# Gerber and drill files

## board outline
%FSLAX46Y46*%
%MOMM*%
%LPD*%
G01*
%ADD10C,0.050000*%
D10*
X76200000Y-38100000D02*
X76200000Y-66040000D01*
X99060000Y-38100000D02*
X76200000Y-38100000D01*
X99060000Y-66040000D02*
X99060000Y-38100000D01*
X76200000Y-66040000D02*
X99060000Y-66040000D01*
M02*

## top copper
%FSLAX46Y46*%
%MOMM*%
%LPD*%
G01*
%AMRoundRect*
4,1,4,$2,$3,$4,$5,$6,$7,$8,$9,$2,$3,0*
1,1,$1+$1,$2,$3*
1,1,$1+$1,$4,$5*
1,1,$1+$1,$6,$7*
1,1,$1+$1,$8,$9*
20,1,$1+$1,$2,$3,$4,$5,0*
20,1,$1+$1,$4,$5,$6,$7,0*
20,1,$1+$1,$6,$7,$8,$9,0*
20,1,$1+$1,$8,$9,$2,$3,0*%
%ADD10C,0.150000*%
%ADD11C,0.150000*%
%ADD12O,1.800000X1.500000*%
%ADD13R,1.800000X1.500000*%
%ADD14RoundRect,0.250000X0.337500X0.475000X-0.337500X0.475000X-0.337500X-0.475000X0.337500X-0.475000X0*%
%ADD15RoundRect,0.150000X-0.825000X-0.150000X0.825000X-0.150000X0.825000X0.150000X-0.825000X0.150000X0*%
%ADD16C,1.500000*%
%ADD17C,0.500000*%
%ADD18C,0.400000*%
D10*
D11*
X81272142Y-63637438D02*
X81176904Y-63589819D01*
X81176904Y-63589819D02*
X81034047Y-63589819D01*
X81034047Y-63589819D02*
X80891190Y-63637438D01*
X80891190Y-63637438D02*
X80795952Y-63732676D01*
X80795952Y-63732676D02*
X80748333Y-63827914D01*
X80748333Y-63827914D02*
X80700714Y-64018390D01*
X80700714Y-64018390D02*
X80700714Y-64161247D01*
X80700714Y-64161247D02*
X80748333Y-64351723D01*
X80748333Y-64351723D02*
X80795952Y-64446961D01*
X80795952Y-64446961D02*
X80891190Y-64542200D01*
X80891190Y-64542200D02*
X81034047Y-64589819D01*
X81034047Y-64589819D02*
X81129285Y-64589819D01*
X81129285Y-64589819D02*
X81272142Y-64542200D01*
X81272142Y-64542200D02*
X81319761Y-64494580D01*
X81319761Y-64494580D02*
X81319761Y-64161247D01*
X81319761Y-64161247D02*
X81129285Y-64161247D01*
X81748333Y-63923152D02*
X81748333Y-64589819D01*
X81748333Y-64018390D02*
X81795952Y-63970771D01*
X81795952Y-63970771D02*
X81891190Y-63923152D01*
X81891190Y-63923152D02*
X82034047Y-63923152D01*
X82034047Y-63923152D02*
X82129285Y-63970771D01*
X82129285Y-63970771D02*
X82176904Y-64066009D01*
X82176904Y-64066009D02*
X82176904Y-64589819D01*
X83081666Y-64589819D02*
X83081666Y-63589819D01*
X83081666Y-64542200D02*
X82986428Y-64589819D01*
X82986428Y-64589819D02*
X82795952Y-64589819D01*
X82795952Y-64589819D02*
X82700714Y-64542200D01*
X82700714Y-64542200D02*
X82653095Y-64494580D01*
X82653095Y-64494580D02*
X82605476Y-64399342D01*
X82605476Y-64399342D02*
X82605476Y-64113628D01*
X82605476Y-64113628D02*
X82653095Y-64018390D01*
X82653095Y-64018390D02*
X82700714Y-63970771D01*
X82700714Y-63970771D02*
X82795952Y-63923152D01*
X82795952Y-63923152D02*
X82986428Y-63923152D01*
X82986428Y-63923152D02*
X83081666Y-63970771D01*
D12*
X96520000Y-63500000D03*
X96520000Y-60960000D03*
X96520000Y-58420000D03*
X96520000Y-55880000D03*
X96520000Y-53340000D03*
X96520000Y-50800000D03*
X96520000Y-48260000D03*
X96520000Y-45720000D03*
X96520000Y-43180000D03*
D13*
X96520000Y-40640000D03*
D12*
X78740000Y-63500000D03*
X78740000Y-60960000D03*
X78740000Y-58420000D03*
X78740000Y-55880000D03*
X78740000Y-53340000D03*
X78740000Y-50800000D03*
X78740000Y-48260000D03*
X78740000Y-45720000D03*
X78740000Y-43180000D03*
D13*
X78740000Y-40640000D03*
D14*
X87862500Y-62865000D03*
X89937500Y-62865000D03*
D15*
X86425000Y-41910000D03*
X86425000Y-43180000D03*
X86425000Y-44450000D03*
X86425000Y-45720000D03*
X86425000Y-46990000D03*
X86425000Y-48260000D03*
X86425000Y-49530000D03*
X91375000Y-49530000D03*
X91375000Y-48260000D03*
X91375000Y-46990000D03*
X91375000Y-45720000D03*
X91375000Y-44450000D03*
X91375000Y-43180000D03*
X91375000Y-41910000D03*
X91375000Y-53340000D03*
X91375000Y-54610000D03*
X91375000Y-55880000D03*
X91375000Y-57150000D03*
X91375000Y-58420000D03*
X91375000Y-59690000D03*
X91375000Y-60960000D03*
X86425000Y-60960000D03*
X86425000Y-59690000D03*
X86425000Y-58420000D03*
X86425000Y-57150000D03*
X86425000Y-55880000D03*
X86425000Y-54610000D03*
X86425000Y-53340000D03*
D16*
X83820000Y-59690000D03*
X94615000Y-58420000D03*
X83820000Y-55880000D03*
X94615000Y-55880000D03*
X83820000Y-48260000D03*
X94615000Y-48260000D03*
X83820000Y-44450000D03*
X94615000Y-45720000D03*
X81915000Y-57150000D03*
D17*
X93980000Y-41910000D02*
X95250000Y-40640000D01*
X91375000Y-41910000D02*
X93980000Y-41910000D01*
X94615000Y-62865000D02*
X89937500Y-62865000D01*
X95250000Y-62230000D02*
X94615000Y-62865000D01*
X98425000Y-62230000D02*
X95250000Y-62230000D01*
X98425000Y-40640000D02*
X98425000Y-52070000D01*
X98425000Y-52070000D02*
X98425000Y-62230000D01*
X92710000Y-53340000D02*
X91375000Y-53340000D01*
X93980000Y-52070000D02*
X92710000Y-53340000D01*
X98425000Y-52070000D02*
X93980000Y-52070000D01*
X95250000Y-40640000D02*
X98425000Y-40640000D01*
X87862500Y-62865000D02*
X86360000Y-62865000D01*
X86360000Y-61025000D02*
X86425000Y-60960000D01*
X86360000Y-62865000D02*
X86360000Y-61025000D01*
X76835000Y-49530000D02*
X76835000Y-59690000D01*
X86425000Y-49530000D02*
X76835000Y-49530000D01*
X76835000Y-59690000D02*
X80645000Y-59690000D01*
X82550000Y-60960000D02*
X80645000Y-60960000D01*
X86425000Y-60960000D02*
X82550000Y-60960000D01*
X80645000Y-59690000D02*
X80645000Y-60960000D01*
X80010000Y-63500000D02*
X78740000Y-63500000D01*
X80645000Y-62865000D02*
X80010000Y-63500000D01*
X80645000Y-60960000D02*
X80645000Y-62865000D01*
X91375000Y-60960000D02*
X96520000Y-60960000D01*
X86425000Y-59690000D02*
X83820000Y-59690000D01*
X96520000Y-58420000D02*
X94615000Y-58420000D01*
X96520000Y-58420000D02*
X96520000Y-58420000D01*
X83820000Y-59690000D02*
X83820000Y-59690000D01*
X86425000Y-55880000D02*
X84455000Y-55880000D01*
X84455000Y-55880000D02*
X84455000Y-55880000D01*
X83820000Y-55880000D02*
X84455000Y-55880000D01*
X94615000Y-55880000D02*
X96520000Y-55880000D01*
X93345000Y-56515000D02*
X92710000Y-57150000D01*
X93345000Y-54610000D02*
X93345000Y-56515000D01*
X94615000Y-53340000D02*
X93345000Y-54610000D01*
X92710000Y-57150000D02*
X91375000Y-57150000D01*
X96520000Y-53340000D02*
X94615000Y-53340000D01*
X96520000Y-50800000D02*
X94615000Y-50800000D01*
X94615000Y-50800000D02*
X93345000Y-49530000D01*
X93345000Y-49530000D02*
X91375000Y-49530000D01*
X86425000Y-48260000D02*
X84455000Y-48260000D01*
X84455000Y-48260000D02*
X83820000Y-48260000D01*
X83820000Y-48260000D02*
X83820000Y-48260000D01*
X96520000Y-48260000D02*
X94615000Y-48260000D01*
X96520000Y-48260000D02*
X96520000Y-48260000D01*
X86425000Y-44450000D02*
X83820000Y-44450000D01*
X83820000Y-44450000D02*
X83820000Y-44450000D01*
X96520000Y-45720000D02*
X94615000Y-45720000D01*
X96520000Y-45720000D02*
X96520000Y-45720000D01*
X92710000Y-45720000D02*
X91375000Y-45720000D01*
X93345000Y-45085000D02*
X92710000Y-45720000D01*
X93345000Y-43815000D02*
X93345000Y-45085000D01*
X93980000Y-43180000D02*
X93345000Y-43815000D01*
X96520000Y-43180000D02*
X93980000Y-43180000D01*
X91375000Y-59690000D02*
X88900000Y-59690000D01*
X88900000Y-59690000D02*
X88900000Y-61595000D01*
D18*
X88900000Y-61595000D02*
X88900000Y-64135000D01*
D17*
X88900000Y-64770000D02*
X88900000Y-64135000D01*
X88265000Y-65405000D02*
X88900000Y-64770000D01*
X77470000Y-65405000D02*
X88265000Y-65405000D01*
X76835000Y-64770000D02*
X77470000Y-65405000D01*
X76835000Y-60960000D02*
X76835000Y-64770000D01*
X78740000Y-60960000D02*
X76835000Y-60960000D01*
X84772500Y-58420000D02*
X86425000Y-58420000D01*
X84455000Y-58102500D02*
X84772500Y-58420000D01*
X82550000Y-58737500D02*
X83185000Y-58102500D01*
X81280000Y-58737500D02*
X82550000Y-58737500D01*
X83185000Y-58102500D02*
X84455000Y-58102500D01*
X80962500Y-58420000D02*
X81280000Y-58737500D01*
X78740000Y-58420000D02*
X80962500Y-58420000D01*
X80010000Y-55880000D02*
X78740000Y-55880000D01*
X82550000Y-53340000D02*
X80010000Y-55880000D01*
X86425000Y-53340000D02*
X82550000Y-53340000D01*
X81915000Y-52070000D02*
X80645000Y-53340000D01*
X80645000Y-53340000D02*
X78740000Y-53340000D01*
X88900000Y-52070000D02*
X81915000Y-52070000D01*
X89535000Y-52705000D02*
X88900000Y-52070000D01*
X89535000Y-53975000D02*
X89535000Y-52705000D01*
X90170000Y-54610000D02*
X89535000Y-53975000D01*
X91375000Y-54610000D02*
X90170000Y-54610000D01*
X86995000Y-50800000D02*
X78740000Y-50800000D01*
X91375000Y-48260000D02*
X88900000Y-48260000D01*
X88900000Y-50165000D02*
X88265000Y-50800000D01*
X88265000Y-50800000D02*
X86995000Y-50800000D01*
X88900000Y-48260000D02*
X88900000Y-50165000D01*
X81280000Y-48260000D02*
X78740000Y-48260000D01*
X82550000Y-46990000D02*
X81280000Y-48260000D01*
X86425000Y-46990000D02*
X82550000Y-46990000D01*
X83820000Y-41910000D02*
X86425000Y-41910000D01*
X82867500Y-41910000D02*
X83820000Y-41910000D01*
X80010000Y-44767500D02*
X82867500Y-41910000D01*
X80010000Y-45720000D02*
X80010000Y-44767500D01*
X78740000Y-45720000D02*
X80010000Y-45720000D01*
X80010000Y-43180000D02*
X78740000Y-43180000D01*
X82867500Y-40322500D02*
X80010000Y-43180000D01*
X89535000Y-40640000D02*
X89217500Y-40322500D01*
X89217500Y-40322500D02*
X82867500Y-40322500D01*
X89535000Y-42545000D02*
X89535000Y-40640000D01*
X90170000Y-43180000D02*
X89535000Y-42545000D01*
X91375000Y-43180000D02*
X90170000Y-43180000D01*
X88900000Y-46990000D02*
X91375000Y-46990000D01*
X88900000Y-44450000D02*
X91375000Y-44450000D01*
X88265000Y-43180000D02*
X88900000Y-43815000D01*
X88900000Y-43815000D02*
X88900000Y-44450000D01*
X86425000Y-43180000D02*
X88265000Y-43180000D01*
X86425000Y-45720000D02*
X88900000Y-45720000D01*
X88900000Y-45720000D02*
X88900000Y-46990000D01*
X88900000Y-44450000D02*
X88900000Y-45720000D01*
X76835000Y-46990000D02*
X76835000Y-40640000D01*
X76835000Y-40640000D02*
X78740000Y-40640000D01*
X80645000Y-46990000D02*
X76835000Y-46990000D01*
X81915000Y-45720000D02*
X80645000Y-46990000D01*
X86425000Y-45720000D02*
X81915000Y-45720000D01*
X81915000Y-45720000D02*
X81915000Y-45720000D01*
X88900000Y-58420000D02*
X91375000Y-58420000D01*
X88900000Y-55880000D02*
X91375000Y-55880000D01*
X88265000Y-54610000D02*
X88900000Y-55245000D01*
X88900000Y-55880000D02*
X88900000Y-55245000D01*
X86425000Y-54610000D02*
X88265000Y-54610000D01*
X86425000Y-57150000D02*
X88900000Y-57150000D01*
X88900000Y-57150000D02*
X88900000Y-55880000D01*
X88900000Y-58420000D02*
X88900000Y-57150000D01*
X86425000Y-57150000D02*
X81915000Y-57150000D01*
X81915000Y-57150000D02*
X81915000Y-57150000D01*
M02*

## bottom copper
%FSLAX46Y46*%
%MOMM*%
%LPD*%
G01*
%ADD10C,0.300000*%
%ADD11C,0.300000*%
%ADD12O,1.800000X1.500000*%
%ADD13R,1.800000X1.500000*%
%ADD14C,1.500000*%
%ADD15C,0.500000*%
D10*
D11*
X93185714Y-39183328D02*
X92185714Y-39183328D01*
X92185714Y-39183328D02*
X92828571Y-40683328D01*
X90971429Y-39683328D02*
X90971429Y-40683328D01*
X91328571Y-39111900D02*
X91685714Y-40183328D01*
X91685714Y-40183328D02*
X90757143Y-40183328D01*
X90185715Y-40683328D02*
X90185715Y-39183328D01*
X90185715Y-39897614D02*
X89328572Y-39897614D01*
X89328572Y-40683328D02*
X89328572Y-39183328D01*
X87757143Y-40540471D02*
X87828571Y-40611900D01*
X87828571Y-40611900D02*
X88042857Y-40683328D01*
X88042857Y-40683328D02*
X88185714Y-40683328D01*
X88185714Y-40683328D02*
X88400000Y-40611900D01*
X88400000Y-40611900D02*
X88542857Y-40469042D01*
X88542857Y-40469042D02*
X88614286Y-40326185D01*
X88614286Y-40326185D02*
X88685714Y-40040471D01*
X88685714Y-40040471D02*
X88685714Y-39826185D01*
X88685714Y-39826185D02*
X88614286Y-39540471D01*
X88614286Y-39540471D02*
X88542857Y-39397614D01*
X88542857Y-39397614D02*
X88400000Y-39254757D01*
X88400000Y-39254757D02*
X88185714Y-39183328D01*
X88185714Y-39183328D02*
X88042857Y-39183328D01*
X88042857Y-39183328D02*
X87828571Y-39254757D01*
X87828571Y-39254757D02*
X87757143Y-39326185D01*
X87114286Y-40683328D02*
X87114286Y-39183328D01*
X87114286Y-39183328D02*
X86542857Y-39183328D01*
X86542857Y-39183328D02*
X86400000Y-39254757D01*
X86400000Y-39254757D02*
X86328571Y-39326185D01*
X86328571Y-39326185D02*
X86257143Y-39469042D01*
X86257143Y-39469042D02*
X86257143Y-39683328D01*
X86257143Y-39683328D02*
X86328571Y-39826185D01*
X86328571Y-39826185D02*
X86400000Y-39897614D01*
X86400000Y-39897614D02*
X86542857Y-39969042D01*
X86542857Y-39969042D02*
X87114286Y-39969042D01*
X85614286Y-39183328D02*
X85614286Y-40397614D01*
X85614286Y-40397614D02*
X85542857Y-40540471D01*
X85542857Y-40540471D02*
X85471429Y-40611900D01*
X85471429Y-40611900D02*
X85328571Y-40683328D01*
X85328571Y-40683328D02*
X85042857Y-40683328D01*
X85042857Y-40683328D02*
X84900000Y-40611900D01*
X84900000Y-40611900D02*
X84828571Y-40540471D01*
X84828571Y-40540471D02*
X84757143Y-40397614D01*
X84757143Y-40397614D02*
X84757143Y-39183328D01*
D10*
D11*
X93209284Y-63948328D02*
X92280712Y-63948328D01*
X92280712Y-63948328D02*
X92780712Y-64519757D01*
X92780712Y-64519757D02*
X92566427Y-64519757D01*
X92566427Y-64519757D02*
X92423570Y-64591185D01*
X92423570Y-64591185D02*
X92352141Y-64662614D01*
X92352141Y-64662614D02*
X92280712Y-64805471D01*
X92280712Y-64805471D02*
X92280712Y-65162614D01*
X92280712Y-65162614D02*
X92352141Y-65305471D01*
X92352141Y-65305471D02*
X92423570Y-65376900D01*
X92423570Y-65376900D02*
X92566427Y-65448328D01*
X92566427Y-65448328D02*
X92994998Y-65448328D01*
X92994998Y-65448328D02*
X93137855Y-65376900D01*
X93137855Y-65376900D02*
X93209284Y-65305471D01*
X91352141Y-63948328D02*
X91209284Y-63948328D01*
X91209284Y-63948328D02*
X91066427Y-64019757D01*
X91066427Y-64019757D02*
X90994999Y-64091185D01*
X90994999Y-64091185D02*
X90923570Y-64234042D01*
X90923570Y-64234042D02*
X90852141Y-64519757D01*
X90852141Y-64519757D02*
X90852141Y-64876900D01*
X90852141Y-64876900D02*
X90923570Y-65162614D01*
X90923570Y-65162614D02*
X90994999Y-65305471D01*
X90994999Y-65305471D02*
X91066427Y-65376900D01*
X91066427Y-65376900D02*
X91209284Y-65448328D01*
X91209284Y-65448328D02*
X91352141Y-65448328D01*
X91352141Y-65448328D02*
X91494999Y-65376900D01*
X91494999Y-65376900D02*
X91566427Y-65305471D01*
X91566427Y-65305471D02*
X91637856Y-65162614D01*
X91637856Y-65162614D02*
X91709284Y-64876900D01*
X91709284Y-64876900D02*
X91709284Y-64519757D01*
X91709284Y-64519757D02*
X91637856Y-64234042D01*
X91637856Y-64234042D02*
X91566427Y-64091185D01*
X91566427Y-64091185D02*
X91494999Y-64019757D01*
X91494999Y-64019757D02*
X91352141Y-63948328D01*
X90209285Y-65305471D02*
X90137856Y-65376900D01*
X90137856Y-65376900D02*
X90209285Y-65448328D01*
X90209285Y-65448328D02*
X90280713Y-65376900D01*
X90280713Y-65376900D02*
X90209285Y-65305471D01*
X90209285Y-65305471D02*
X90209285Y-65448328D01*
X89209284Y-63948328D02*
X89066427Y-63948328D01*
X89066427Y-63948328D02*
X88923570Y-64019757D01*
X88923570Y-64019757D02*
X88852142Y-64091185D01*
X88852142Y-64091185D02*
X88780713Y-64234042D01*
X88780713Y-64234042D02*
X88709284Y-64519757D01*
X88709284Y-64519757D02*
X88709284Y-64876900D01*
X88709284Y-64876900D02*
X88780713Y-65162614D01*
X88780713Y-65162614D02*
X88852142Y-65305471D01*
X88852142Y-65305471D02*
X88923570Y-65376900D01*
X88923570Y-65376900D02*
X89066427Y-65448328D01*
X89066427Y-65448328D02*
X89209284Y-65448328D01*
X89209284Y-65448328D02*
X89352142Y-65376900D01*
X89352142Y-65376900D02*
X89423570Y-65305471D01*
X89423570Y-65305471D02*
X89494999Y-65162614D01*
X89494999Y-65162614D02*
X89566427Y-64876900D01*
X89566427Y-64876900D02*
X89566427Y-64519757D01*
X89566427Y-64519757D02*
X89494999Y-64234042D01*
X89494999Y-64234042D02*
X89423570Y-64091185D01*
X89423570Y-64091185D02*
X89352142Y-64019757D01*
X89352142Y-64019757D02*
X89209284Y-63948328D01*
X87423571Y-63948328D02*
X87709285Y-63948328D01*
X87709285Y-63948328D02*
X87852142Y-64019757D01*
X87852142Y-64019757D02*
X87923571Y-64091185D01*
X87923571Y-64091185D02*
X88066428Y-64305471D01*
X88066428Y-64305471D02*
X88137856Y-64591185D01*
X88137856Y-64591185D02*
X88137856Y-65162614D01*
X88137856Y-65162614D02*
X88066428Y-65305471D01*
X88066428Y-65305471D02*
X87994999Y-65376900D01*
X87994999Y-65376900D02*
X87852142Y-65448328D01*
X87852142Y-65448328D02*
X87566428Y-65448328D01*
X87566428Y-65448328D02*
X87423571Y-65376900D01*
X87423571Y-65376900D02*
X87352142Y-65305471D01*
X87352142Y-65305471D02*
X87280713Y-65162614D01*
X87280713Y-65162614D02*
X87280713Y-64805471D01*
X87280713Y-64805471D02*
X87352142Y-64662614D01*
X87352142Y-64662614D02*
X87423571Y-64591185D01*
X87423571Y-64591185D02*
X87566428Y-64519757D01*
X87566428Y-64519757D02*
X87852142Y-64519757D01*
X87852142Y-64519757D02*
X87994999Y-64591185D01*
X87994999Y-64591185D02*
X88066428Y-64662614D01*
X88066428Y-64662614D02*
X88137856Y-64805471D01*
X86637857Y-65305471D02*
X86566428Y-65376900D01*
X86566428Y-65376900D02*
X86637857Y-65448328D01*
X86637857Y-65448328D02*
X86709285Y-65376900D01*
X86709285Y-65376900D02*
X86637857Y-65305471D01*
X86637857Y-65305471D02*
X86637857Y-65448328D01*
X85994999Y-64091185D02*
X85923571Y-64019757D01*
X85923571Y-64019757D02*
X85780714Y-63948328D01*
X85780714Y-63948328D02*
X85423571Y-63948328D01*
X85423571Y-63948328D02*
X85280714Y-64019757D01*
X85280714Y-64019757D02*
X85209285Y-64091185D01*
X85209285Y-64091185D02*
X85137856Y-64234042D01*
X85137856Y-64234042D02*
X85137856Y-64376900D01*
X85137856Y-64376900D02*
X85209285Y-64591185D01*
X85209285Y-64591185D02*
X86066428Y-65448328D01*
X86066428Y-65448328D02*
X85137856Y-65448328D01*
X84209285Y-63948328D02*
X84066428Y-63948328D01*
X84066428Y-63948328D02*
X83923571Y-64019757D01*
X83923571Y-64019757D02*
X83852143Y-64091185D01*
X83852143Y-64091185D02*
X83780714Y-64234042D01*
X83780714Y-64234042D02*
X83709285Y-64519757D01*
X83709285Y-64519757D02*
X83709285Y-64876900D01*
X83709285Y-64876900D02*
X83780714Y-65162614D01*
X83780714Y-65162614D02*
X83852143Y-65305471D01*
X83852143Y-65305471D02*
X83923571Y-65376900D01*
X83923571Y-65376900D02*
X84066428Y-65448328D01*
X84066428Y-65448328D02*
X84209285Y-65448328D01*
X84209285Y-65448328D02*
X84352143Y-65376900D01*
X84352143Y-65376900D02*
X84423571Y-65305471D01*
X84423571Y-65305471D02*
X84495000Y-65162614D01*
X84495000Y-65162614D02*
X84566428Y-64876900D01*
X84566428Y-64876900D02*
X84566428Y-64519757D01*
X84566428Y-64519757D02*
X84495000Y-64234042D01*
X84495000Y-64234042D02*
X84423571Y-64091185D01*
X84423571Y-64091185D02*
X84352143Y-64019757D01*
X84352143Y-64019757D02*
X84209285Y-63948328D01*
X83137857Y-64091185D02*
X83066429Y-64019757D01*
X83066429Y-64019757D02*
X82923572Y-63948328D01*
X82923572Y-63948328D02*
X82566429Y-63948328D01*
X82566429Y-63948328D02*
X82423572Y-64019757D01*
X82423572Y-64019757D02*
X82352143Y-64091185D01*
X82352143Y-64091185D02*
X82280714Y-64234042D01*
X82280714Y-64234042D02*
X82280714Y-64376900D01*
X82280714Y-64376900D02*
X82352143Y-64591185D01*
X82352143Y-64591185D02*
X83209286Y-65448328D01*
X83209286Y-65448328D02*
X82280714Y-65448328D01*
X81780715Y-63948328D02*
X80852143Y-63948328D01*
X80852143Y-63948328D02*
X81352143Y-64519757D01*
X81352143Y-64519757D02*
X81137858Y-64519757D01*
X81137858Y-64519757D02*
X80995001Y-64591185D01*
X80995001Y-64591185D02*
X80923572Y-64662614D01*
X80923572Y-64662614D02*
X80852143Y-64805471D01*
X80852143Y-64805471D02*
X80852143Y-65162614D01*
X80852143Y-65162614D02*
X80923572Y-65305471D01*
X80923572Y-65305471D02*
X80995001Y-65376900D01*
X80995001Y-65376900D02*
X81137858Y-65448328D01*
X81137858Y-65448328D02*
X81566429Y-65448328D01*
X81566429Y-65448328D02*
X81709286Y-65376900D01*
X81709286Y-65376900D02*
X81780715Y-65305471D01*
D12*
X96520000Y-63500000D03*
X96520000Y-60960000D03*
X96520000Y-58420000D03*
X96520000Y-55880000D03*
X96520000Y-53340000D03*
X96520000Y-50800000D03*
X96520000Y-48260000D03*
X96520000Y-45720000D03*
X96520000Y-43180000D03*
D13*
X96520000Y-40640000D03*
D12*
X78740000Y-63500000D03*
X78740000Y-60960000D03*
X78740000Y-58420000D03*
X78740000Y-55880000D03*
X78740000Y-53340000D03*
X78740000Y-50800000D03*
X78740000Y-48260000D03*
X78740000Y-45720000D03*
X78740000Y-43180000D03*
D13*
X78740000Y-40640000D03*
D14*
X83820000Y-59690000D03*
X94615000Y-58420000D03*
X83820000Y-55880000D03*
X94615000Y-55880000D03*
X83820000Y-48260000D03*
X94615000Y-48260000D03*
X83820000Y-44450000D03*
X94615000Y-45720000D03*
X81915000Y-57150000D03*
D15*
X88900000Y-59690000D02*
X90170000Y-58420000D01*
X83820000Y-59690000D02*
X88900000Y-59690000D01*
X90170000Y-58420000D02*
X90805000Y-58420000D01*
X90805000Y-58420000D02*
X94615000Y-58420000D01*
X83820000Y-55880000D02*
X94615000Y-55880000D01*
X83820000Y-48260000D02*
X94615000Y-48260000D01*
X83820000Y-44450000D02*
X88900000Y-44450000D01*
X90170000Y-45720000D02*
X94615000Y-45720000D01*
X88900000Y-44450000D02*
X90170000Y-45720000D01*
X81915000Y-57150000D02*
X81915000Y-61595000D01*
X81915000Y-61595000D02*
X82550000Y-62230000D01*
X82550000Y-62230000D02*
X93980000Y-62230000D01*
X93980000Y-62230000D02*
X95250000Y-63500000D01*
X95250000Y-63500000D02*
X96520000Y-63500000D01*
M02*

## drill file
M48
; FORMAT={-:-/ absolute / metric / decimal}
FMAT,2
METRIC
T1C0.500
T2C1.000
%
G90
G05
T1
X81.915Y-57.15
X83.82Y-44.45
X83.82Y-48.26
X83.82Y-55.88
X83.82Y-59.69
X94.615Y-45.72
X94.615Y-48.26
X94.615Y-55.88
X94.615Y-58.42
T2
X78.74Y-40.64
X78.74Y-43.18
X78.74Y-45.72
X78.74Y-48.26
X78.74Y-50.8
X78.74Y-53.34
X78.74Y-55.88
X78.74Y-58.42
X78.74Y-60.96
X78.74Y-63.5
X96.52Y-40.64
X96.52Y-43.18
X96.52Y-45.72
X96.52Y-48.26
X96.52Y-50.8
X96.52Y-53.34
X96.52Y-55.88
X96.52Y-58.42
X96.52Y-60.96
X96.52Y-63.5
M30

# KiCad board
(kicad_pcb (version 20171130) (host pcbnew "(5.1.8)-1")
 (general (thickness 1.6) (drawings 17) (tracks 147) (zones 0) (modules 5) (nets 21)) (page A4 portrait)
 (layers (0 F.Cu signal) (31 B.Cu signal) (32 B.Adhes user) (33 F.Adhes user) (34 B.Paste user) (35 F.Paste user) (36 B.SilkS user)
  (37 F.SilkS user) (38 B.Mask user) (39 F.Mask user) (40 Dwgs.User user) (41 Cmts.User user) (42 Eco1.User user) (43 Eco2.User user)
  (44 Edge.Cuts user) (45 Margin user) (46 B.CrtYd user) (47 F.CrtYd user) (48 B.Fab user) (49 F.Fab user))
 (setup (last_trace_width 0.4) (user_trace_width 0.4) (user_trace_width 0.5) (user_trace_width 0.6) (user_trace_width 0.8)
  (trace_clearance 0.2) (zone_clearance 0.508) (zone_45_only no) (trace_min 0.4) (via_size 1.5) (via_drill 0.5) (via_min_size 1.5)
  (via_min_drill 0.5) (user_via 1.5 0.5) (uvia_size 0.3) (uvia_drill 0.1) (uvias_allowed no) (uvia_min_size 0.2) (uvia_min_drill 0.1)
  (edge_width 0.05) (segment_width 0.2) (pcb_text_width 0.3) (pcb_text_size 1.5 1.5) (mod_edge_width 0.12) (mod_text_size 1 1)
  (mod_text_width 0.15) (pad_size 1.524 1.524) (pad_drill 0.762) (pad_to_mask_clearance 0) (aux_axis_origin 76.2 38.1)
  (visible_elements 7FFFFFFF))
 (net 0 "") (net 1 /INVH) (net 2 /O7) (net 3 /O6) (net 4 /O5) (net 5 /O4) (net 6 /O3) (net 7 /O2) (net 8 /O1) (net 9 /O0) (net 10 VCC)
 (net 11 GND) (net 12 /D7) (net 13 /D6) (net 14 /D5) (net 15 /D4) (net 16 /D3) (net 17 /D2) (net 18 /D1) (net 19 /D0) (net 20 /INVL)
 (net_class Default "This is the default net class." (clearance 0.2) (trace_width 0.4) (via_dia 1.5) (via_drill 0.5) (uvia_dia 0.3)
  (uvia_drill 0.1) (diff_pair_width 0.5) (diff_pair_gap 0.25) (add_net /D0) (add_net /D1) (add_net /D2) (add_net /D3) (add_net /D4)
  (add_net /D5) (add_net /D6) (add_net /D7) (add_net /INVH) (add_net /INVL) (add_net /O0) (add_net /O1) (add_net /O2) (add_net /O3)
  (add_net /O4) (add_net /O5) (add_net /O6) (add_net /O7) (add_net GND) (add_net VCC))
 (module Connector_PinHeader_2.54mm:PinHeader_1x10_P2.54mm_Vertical (layer B.Cu) (at 96.52 40.64 180)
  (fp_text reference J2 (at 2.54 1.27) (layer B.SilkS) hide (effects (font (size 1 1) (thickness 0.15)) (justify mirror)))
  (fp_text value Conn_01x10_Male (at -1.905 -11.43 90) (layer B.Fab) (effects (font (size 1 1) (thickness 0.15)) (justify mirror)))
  (pad 10 thru_hole oval (at 0 -22.86 180) (size 1.8 1.5) (drill 1) (layers *.Cu *.Mask) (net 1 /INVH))
  (pad 9 thru_hole oval (at 0 -20.32 180) (size 1.8 1.5) (drill 1) (layers *.Cu *.Mask) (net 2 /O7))
  (pad 8 thru_hole oval (at 0 -17.78 180) (size 1.8 1.5) (drill 1) (layers *.Cu *.Mask) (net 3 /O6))
  (pad 7 thru_hole oval (at 0 -15.24 180) (size 1.8 1.5) (drill 1) (layers *.Cu *.Mask) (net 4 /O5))
  (pad 6 thru_hole oval (at 0 -12.7 180) (size 1.8 1.5) (drill 1) (layers *.Cu *.Mask) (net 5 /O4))
  (pad 5 thru_hole oval (at 0 -10.16 180) (size 1.8 1.5) (drill 1) (layers *.Cu *.Mask) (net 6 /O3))
  (pad 4 thru_hole oval (at 0 -7.62 180) (size 1.8 1.5) (drill 1) (layers *.Cu *.Mask) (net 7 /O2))
  (pad 3 thru_hole oval (at 0 -5.08 180) (size 1.8 1.5) (drill 1) (layers *.Cu *.Mask) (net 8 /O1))
  (pad 2 thru_hole oval (at 0 -2.54 180) (size 1.8 1.5) (drill 1) (layers *.Cu *.Mask) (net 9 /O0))
  (pad 1 thru_hole rect (at 0 0 180) (size 1.8 1.5) (drill 1) (layers *.Cu *.Mask) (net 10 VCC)))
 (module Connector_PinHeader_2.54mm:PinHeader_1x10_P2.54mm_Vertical (layer B.Cu) (at 78.74 40.64 180)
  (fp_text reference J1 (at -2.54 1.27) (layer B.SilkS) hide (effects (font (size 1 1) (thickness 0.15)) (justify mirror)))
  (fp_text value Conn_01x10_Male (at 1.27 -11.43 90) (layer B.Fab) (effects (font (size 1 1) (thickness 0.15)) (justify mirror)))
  (pad 10 thru_hole oval (at 0 -22.86 180) (size 1.8 1.5) (drill 1) (layers *.Cu *.Mask) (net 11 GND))
  (pad 9 thru_hole oval (at 0 -20.32 180) (size 1.8 1.5) (drill 1) (layers *.Cu *.Mask) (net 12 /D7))
  (pad 8 thru_hole oval (at 0 -17.78 180) (size 1.8 1.5) (drill 1) (layers *.Cu *.Mask) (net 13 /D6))
  (pad 7 thru_hole oval (at 0 -15.24 180) (size 1.8 1.5) (drill 1) (layers *.Cu *.Mask) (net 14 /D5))
  (pad 6 thru_hole oval (at 0 -12.7 180) (size 1.8 1.5) (drill 1) (layers *.Cu *.Mask) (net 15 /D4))
  (pad 5 thru_hole oval (at 0 -10.16 180) (size 1.8 1.5) (drill 1) (layers *.Cu *.Mask) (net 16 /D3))
  (pad 4 thru_hole oval (at 0 -7.62 180) (size 1.8 1.5) (drill 1) (layers *.Cu *.Mask) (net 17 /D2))
  (pad 3 thru_hole oval (at 0 -5.08 180) (size 1.8 1.5) (drill 1) (layers *.Cu *.Mask) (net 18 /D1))
  (pad 2 thru_hole oval (at 0 -2.54 180) (size 1.8 1.5) (drill 1) (layers *.Cu *.Mask) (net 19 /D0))
  (pad 1 thru_hole rect (at 0 0 180) (size 1.8 1.5) (drill 1) (layers *.Cu *.Mask) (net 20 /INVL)))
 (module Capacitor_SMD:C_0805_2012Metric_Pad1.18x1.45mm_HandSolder (layer F.Cu) (at 88.9 62.865 180)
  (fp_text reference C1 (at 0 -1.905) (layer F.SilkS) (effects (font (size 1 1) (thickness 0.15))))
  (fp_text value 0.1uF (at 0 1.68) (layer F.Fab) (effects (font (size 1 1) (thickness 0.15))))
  (pad 2 smd roundrect (at 1.0375 0 180) (size 1.175 1.45) (layers F.Cu F.Paste F.Mask) (roundrect_rratio 0.2127659574468085) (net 11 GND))
  (pad 1 smd roundrect (at -1.0375 0 180) (size 1.175 1.45) (layers F.Cu F.Paste F.Mask) (roundrect_rratio 0.2127659574468085) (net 10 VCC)))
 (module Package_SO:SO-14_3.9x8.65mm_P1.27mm (layer F.Cu) (at 88.9 45.72)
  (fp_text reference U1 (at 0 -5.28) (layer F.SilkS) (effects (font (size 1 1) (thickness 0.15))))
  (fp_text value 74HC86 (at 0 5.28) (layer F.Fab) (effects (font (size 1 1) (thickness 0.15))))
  (pad 1 smd roundrect (at -2.475 -3.81) (size 1.95 0.6) (layers F.Cu F.Paste F.Mask) (roundrect_rratio 0.25) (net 18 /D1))
  (pad 2 smd roundrect (at -2.475 -2.54) (size 1.95 0.6) (layers F.Cu F.Paste F.Mask) (roundrect_rratio 0.25) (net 20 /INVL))
  (pad 3 smd roundrect (at -2.475 -1.27) (size 1.95 0.6) (layers F.Cu F.Paste F.Mask) (roundrect_rratio 0.25) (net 8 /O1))
  (pad 4 smd roundrect (at -2.475 0) (size 1.95 0.6) (layers F.Cu F.Paste F.Mask) (roundrect_rratio 0.25) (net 20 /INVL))
  (pad 5 smd roundrect (at -2.475 1.27) (size 1.95 0.6) (layers F.Cu F.Paste F.Mask) (roundrect_rratio 0.25) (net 17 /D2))
  (pad 6 smd roundrect (at -2.475 2.54) (size 1.95 0.6) (layers F.Cu F.Paste F.Mask) (roundrect_rratio 0.25) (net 7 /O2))
  (pad 7 smd roundrect (at -2.475 3.81) (size 1.95 0.6) (layers F.Cu F.Paste F.Mask) (roundrect_rratio 0.25) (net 11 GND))
  (pad 8 smd roundrect (at 2.475 3.81) (size 1.95 0.6) (layers F.Cu F.Paste F.Mask) (roundrect_rratio 0.25) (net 6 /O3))
  (pad 9 smd roundrect (at 2.475 2.54) (size 1.95 0.6) (layers F.Cu F.Paste F.Mask) (roundrect_rratio 0.25) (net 16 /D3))
  (pad 10 smd roundrect (at 2.475 1.27) (size 1.95 0.6) (layers F.Cu F.Paste F.Mask) (roundrect_rratio 0.25) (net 20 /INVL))
  (pad 11 smd roundrect (at 2.475 0) (size 1.95 0.6) (layers F.Cu F.Paste F.Mask) (roundrect_rratio 0.25) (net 9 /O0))
  (pad 12 smd roundrect (at 2.475 -1.27) (size 1.95 0.6) (layers F.Cu F.Paste F.Mask) (roundrect_rratio 0.25) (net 20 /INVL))
  (pad 13 smd roundrect (at 2.475 -2.54) (size 1.95 0.6) (layers F.Cu F.Paste F.Mask) (roundrect_rratio 0.25) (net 19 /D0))
  (pad 14 smd roundrect (at 2.475 -3.81) (size 1.95 0.6) (layers F.Cu F.Paste F.Mask) (roundrect_rratio 0.25) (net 10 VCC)))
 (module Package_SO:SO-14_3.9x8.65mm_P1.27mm (layer F.Cu) (at 88.9 57.15)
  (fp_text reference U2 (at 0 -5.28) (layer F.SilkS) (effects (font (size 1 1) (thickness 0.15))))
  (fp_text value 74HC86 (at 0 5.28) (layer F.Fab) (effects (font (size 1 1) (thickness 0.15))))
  (pad 14 smd roundrect (at 2.475 -3.81) (size 1.95 0.6) (layers F.Cu F.Paste F.Mask) (roundrect_rratio 0.25) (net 10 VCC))
  (pad 13 smd roundrect (at 2.475 -2.54) (size 1.95 0.6) (layers F.Cu F.Paste F.Mask) (roundrect_rratio 0.25) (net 15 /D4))
  (pad 12 smd roundrect (at 2.475 -1.27) (size 1.95 0.6) (layers F.Cu F.Paste F.Mask) (roundrect_rratio 0.25) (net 1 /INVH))
  (pad 11 smd roundrect (at 2.475 0) (size 1.95 0.6) (layers F.Cu F.Paste F.Mask) (roundrect_rratio 0.25) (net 5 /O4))
  (pad 10 smd roundrect (at 2.475 1.27) (size 1.95 0.6) (layers F.Cu F.Paste F.Mask) (roundrect_rratio 0.25) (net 1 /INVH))
  (pad 9 smd roundrect (at 2.475 2.54) (size 1.95 0.6) (layers F.Cu F.Paste F.Mask) (roundrect_rratio 0.25) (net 12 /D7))
  (pad 8 smd roundrect (at 2.475 3.81) (size 1.95 0.6) (layers F.Cu F.Paste F.Mask) (roundrect_rratio 0.25) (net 2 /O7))
  (pad 7 smd roundrect (at -2.475 3.81) (size 1.95 0.6) (layers F.Cu F.Paste F.Mask) (roundrect_rratio 0.25) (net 11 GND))
  (pad 6 smd roundrect (at -2.475 2.54) (size 1.95 0.6) (layers F.Cu F.Paste F.Mask) (roundrect_rratio 0.25) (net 3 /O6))
  (pad 5 smd roundrect (at -2.475 1.27) (size 1.95 0.6) (layers F.Cu F.Paste F.Mask) (roundrect_rratio 0.25) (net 13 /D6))
  (pad 4 smd roundrect (at -2.475 0) (size 1.95 0.6) (layers F.Cu F.Paste F.Mask) (roundrect_rratio 0.25) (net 1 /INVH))
  (pad 3 smd roundrect (at -2.475 -1.27) (size 1.95 0.6) (layers F.Cu F.Paste F.Mask) (roundrect_rratio 0.25) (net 4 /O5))
  (pad 2 smd roundrect (at -2.475 -2.54) (size 1.95 0.6) (layers F.Cu F.Paste F.Mask) (roundrect_rratio 0.25) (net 1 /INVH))
  (pad 1 smd roundrect (at -2.475 -3.81) (size 1.95 0.6) (layers F.Cu F.Paste F.Mask) (roundrect_rratio 0.25) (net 14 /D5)))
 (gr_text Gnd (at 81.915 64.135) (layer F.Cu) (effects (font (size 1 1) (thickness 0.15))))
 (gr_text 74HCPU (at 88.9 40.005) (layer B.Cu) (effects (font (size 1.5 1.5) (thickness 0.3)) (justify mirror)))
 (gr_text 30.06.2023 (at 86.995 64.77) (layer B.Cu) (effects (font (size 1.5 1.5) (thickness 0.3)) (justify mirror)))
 (gr_line (start 76.2 38.1) (end 76.2 66.04) (layer Edge.Cuts) (width 0.05))
 (gr_line (start 99.06 38.1) (end 76.2 38.1) (layer Edge.Cuts) (width 0.05))
 (gr_line (start 99.06 66.04) (end 99.06 38.1) (layer Edge.Cuts) (width 0.05))
 (gr_line (start 76.2 66.04) (end 99.06 66.04) (layer Edge.Cuts) (width 0.05))
 (segment (start 93.98 41.91) (end 95.25 40.64) (width 0.5) (layer F.Cu) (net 10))
 (segment (start 91.375 41.91) (end 93.98 41.91) (width 0.5) (layer F.Cu) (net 10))
 (segment (start 94.615 62.865) (end 89.9375 62.865) (width 0.5) (layer F.Cu) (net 10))
 (segment (start 95.25 62.23) (end 94.615 62.865) (width 0.5) (layer F.Cu) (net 10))
 (segment (start 98.425 62.23) (end 95.25 62.23) (width 0.5) (layer F.Cu) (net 10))
 (segment (start 98.425 40.64) (end 98.425 52.07) (width 0.5) (layer F.Cu) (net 10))
 (segment (start 98.425 52.07) (end 98.425 62.23) (width 0.5) (layer F.Cu) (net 10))
 (segment (start 92.71 53.34) (end 91.375 53.34) (width 0.5) (layer F.Cu) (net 10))
 (segment (start 93.98 52.07) (end 92.71 53.34) (width 0.5) (layer F.Cu) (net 10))
 (segment (start 98.425 52.07) (end 93.98 52.07) (width 0.5) (layer F.Cu) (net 10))
 (segment (start 95.25 40.64) (end 98.425 40.64) (width 0.5) (layer F.Cu) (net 10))
 (segment (start 87.8625 62.865) (end 86.36 62.865) (width 0.5) (layer F.Cu) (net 11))
 (segment (start 86.36 61.025) (end 86.425 60.96) (width 0.5) (layer F.Cu) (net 11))
 (segment (start 86.36 62.865) (end 86.36 61.025) (width 0.5) (layer F.Cu) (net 11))
 (segment (start 76.835 49.53) (end 76.835 59.69) (width 0.5) (layer F.Cu) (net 11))
 (segment (start 86.425 49.53) (end 76.835 49.53) (width 0.5) (layer F.Cu) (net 11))
 (segment (start 76.835 59.69) (end 80.645 59.69) (width 0.5) (layer F.Cu) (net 11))
 (segment (start 82.55 60.96) (end 80.645 60.96) (width 0.5) (layer F.Cu) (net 11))
 (segment (start 86.425 60.96) (end 82.55 60.96) (width 0.5) (layer F.Cu) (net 11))
 (segment (start 80.645 59.69) (end 80.645 60.96) (width 0.5) (layer F.Cu) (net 11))
 (segment (start 80.01 63.5) (end 78.74 63.5) (width 0.5) (layer F.Cu) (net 11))
 (segment (start 80.645 62.865) (end 80.01 63.5) (width 0.5) (layer F.Cu) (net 11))
 (segment (start 80.645 60.96) (end 80.645 62.865) (width 0.5) (layer F.Cu) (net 11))
 (segment (start 91.375 60.96) (end 96.52 60.96) (width 0.5) (layer F.Cu) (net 2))
 (segment (start 86.425 59.69) (end 83.82 59.69) (width 0.5) (layer F.Cu) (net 3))
 (segment (start 96.52 58.42) (end 94.615 58.42) (width 0.5) (layer F.Cu) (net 3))
 (segment (start 96.52 58.42) (end 96.52 58.42) (width 0.5) (layer F.Cu) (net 3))
 (segment (start 83.82 59.69) (end 83.82 59.69) (width 0.5) (layer F.Cu) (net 3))
 (via (at 83.82 59.69) (size 1.5) (drill 0.5) (layers F.Cu B.Cu) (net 3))
 (segment (start 88.9 59.69) (end 90.17 58.42) (width 0.5) (layer B.Cu) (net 3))
 (segment (start 83.82 59.69) (end 88.9 59.69) (width 0.5) (layer B.Cu) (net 3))
 (segment (start 90.17 58.42) (end 90.805 58.42) (width 0.5) (layer B.Cu) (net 3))
 (segment (start 90.805 58.42) (end 94.615 58.42) (width 0.5) (layer B.Cu) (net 3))
 (via (at 94.615 58.42) (size 1.5) (drill 0.5) (layers F.Cu B.Cu) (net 3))
 (segment (start 86.425 55.88) (end 84.455 55.88) (width 0.5) (layer F.Cu) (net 4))
 (segment (start 84.455 55.88) (end 84.455 55.88) (width 0.5) (layer F.Cu) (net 4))
 (via (at 83.82 55.88) (size 1.5) (drill 0.5) (layers F.Cu B.Cu) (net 4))
 (segment (start 83.82 55.88) (end 84.455 55.88) (width 0.5) (layer F.Cu) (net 4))
 (segment (start 94.615 55.88) (end 96.52 55.88) (width 0.5) (layer F.Cu) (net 4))
 (segment (start 83.82 55.88) (end 94.615 55.88) (width 0.5) (layer B.Cu) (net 4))
 (via (at 94.615 55.88) (size 1.5) (drill 0.5) (layers F.Cu B.Cu) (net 4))
 (segment (start 93.345 56.515) (end 92.71 57.15) (width 0.5) (layer F.Cu) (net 5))
 (segment (start 93.345 54.61) (end 93.345 56.515) (width 0.5) (layer F.Cu) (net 5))
 (segment (start 94.615 53.34) (end 93.345 54.61) (width 0.5) (layer F.Cu) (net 5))
 (segment (start 92.71 57.15) (end 91.375 57.15) (width 0.5) (layer F.Cu) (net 5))
 (segment (start 96.52 53.34) (end 94.615 53.34) (width 0.5) (layer F.Cu) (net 5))
 (segment (start 96.52 50.8) (end 94.615 50.8) (width 0.5) (layer F.Cu) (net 6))
 (segment (start 94.615 50.8) (end 93.345 49.53) (width 0.5) (layer F.Cu) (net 6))
 (segment (start 93.345 49.53) (end 91.375 49.53) (width 0.5) (layer F.Cu) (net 6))
 (segment (start 86.425 48.26) (end 84.455 48.26) (width 0.5) (layer F.Cu) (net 7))
 (segment (start 84.455 48.26) (end 83.82 48.26) (width 0.5) (layer F.Cu) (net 7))
 (segment (start 83.82 48.26) (end 83.82 48.26) (width 0.5) (layer F.Cu) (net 7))
 (via (at 83.82 48.26) (size 1.5) (drill 0.5) (layers F.Cu B.Cu) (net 7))
 (segment (start 96.52 48.26) (end 94.615 48.26) (width 0.5) (layer F.Cu) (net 7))
 (segment (start 96.52 48.26) (end 96.52 48.26) (width 0.5) (layer F.Cu) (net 7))
 (segment (start 83.82 48.26) (end 94.615 48.26) (width 0.5) (layer B.Cu) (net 7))
 (via (at 94.615 48.26) (size 1.5) (drill 0.5) (layers F.Cu B.Cu) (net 7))
 (segment (start 86.425 44.45) (end 83.82 44.45) (width 0.5) (layer F.Cu) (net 8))
 (segment (start 83.82 44.45) (end 83.82 44.45) (width 0.5) (layer F.Cu) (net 8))
 (via (at 83.82 44.45) (size 1.5) (drill 0.5) (layers F.Cu B.Cu) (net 8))
 (segment (start 96.52 45.72) (end 94.615 45.72) (width 0.5) (layer F.Cu) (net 8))
 (segment (start 96.52 45.72) (end 96.52 45.72) (width 0.5) (layer F.Cu) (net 8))
 (segment (start 83.82 44.45) (end 88.9 44.45) (width 0.5) (layer B.Cu) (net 8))
 (segment (start 90.17 45.72) (end 94.615 45.72) (width 0.5) (layer B.Cu) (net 8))
 (segment (start 88.9 44.45) (end 90.17 45.72) (width 0.5) (layer B.Cu) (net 8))
 (via (at 94.615 45.72) (size 1.5) (drill 0.5) (layers F.Cu B.Cu) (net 8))
 (segment (start 92.71 45.72) (end 91.375 45.72) (width 0.5) (layer F.Cu) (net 9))
 (segment (start 93.345 45.085) (end 92.71 45.72) (width 0.5) (layer F.Cu) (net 9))
 (segment (start 93.345 43.815) (end 93.345 45.085) (width 0.5) (layer F.Cu) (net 9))
 (segment (start 93.98 43.18) (end 93.345 43.815) (width 0.5) (layer F.Cu) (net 9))
 (segment (start 96.52 43.18) (end 93.98 43.18) (width 0.5) (layer F.Cu) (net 9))
 (segment (start 91.375 59.69) (end 88.9 59.69) (width 0.5) (layer F.Cu) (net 12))
 (segment (start 88.9 59.69) (end 88.9 61.595) (width 0.5) (layer F.Cu) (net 12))
 (segment (start 88.9 61.595) (end 88.9 64.135) (width 0.4) (layer F.Cu) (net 12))
 (segment (start 88.9 64.77) (end 88.9 64.135) (width 0.5) (layer F.Cu) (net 12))
 (segment (start 88.265 65.405) (end 88.9 64.77) (width 0.5) (layer F.Cu) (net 12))
 (segment (start 77.47 65.405) (end 88.265 65.405) (width 0.5) (layer F.Cu) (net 12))
 (segment (start 76.835 64.77) (end 77.47 65.405) (width 0.5) (layer F.Cu) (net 12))
 (segment (start 76.835 60.96) (end 76.835 64.77) (width 0.5) (layer F.Cu) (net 12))
 (segment (start 78.74 60.96) (end 76.835 60.96) (width 0.5) (layer F.Cu) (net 12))
 (segment (start 84.7725 58.42) (end 86.425 58.42) (width 0.5) (layer F.Cu) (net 13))
 (segment (start 84.455 58.1025) (end 84.7725 58.42) (width 0.5) (layer F.Cu) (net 13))
 (segment (start 82.55 58.7375) (end 83.185 58.1025) (width 0.5) (layer F.Cu) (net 13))
 (segment (start 81.28 58.7375) (end 82.55 58.7375) (width 0.5) (layer F.Cu) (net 13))
 (segment (start 83.185 58.1025) (end 84.455 58.1025) (width 0.5) (layer F.Cu) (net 13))
 (segment (start 80.9625 58.42) (end 81.28 58.7375) (width 0.5) (layer F.Cu) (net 13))
 (segment (start 78.74 58.42) (end 80.9625 58.42) (width 0.5) (layer F.Cu) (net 13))
 (segment (start 80.01 55.88) (end 78.74 55.88) (width 0.5) (layer F.Cu) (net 14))
 (segment (start 82.55 53.34) (end 80.01 55.88) (width 0.5) (layer F.Cu) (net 14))
 (segment (start 86.425 53.34) (end 82.55 53.34) (width 0.5) (layer F.Cu) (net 14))
 (segment (start 81.915 52.07) (end 80.645 53.34) (width 0.5) (layer F.Cu) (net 15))
 (segment (start 80.645 53.34) (end 78.74 53.34) (width 0.5) (layer F.Cu) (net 15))
 (segment (start 88.9 52.07) (end 81.915 52.07) (width 0.5) (layer F.Cu) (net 15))
 (segment (start 89.535 52.705) (end 88.9 52.07) (width 0.5) (layer F.Cu) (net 15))
 (segment (start 89.535 53.975) (end 89.535 52.705) (width 0.5) (layer F.Cu) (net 15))
 (segment (start 90.17 54.61) (end 89.535 53.975) (width 0.5) (layer F.Cu) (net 15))
 (segment (start 91.375 54.61) (end 90.17 54.61) (width 0.5) (layer F.Cu) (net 15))
 (segment (start 86.995 50.8) (end 78.74 50.8) (width 0.5) (layer F.Cu) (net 16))
 (segment (start 91.375 48.26) (end 88.9 48.26) (width 0.5) (layer F.Cu) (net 16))
 (segment (start 88.9 50.165) (end 88.265 50.8) (width 0.5) (layer F.Cu) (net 16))
 (segment (start 88.265 50.8) (end 86.995 50.8) (width 0.5) (layer F.Cu) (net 16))
 (segment (start 88.9 48.26) (end 88.9 50.165) (width 0.5) (layer F.Cu) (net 16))
 (segment (start 81.28 48.26) (end 78.74 48.26) (width 0.5) (layer F.Cu) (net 17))
 (segment (start 82.55 46.99) (end 81.28 48.26) (width 0.5) (layer F.Cu) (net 17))
 (segment (start 86.425 46.99) (end 82.55 46.99) (width 0.5) (layer F.Cu) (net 17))
 (segment (start 83.82 41.91) (end 86.425 41.91) (width 0.5) (layer F.Cu) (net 18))
 (segment (start 82.8675 41.91) (end 83.82 41.91) (width 0.5) (layer F.Cu) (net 18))
 (segment (start 80.01 44.7675) (end 82.8675 41.91) (width 0.5) (layer F.Cu) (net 18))
 (segment (start 80.01 45.72) (end 80.01 44.7675) (width 0.5) (layer F.Cu) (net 18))
 (segment (start 78.74 45.72) (end 80.01 45.72) (width 0.5) (layer F.Cu) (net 18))
 (segment (start 80.01 43.18) (end 78.74 43.18) (width 0.5) (layer F.Cu) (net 19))
 (segment (start 82.8675 40.3225) (end 80.01 43.18) (width 0.5) (layer F.Cu) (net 19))
 (segment (start 89.535 40.64) (end 89.2175 40.3225) (width 0.5) (layer F.Cu) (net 19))
 (segment (start 89.2175 40.3225) (end 82.8675 40.3225) (width 0.5) (layer F.Cu) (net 19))
 (segment (start 89.535 42.545) (end 89.535 40.64) (width 0.5) (layer F.Cu) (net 19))
 (segment (start 90.17 43.18) (end 89.535 42.545) (width 0.5) (layer F.Cu) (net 19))
 (segment (start 91.375 43.18) (end 90.17 43.18) (width 0.5) (layer F.Cu) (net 19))
 (segment (start 88.9 46.99) (end 91.375 46.99) (width 0.5) (layer F.Cu) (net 20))
 (segment (start 88.9 44.45) (end 91.375 44.45) (width 0.5) (layer F.Cu) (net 20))
 (segment (start 88.265 43.18) (end 88.9 43.815) (width 0.5) (layer F.Cu) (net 20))
 (segment (start 88.9 43.815) (end 88.9 44.45) (width 0.5) (layer F.Cu) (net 20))
 (segment (start 86.425 43.18) (end 88.265 43.18) (width 0.5) (layer F.Cu) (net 20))
 (segment (start 86.425 45.72) (end 88.9 45.72) (width 0.5) (layer F.Cu) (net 20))
 (segment (start 88.9 45.72) (end 88.9 46.99) (width 0.5) (layer F.Cu) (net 20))
 (segment (start 88.9 44.45) (end 88.9 45.72) (width 0.5) (layer F.Cu) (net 20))
 (segment (start 76.835 46.99) (end 76.835 40.64) (width 0.5) (layer F.Cu) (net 20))
 (segment (start 76.835 40.64) (end 78.74 40.64) (width 0.5) (layer F.Cu) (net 20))
 (segment (start 80.645 46.99) (end 76.835 46.99) (width 0.5) (layer F.Cu) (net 20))
 (segment (start 81.915 45.72) (end 80.645 46.99) (width 0.5) (layer F.Cu) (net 20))
 (segment (start 86.425 45.72) (end 81.915 45.72) (width 0.5) (layer F.Cu) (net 20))
 (segment (start 81.915 45.72) (end 81.915 45.72) (width 0.5) (layer F.Cu) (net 20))
 (segment (start 88.9 58.42) (end 91.375 58.42) (width 0.5) (layer F.Cu) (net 1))
 (segment (start 88.9 55.88) (end 91.375 55.88) (width 0.5) (layer F.Cu) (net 1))
 (segment (start 88.265 54.61) (end 88.9 55.245) (width 0.5) (layer F.Cu) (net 1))
 (segment (start 88.9 55.88) (end 88.9 55.245) (width 0.5) (layer F.Cu) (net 1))
 (segment (start 86.425 54.61) (end 88.265 54.61) (width 0.5) (layer F.Cu) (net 1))
 (segment (start 86.425 57.15) (end 88.9 57.15) (width 0.5) (layer F.Cu) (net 1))
 (segment (start 88.9 57.15) (end 88.9 55.88) (width 0.5) (layer F.Cu) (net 1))
 (segment (start 88.9 58.42) (end 88.9 57.15) (width 0.5) (layer F.Cu) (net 1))
 (segment (start 86.425 57.15) (end 81.915 57.15) (width 0.5) (layer F.Cu) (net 1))
 (segment (start 81.915 57.15) (end 81.915 57.15) (width 0.5) (layer F.Cu) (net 1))
 (via (at 81.915 57.15) (size 1.5) (drill 0.5) (layers F.Cu B.Cu) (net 1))
 (segment (start 81.915 57.15) (end 81.915 61.595) (width 0.5) (layer B.Cu) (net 1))
 (segment (start 81.915 61.595) (end 82.55 62.23) (width 0.5) (layer B.Cu) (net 1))
 (segment (start 82.55 62.23) (end 93.98 62.23) (width 0.5) (layer B.Cu) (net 1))
 (segment (start 93.98 62.23) (end 95.25 63.5) (width 0.5) (layer B.Cu) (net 1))
 (segment (start 95.25 63.5) (end 96.52 63.5) (width 0.5) (layer B.Cu) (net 1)))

